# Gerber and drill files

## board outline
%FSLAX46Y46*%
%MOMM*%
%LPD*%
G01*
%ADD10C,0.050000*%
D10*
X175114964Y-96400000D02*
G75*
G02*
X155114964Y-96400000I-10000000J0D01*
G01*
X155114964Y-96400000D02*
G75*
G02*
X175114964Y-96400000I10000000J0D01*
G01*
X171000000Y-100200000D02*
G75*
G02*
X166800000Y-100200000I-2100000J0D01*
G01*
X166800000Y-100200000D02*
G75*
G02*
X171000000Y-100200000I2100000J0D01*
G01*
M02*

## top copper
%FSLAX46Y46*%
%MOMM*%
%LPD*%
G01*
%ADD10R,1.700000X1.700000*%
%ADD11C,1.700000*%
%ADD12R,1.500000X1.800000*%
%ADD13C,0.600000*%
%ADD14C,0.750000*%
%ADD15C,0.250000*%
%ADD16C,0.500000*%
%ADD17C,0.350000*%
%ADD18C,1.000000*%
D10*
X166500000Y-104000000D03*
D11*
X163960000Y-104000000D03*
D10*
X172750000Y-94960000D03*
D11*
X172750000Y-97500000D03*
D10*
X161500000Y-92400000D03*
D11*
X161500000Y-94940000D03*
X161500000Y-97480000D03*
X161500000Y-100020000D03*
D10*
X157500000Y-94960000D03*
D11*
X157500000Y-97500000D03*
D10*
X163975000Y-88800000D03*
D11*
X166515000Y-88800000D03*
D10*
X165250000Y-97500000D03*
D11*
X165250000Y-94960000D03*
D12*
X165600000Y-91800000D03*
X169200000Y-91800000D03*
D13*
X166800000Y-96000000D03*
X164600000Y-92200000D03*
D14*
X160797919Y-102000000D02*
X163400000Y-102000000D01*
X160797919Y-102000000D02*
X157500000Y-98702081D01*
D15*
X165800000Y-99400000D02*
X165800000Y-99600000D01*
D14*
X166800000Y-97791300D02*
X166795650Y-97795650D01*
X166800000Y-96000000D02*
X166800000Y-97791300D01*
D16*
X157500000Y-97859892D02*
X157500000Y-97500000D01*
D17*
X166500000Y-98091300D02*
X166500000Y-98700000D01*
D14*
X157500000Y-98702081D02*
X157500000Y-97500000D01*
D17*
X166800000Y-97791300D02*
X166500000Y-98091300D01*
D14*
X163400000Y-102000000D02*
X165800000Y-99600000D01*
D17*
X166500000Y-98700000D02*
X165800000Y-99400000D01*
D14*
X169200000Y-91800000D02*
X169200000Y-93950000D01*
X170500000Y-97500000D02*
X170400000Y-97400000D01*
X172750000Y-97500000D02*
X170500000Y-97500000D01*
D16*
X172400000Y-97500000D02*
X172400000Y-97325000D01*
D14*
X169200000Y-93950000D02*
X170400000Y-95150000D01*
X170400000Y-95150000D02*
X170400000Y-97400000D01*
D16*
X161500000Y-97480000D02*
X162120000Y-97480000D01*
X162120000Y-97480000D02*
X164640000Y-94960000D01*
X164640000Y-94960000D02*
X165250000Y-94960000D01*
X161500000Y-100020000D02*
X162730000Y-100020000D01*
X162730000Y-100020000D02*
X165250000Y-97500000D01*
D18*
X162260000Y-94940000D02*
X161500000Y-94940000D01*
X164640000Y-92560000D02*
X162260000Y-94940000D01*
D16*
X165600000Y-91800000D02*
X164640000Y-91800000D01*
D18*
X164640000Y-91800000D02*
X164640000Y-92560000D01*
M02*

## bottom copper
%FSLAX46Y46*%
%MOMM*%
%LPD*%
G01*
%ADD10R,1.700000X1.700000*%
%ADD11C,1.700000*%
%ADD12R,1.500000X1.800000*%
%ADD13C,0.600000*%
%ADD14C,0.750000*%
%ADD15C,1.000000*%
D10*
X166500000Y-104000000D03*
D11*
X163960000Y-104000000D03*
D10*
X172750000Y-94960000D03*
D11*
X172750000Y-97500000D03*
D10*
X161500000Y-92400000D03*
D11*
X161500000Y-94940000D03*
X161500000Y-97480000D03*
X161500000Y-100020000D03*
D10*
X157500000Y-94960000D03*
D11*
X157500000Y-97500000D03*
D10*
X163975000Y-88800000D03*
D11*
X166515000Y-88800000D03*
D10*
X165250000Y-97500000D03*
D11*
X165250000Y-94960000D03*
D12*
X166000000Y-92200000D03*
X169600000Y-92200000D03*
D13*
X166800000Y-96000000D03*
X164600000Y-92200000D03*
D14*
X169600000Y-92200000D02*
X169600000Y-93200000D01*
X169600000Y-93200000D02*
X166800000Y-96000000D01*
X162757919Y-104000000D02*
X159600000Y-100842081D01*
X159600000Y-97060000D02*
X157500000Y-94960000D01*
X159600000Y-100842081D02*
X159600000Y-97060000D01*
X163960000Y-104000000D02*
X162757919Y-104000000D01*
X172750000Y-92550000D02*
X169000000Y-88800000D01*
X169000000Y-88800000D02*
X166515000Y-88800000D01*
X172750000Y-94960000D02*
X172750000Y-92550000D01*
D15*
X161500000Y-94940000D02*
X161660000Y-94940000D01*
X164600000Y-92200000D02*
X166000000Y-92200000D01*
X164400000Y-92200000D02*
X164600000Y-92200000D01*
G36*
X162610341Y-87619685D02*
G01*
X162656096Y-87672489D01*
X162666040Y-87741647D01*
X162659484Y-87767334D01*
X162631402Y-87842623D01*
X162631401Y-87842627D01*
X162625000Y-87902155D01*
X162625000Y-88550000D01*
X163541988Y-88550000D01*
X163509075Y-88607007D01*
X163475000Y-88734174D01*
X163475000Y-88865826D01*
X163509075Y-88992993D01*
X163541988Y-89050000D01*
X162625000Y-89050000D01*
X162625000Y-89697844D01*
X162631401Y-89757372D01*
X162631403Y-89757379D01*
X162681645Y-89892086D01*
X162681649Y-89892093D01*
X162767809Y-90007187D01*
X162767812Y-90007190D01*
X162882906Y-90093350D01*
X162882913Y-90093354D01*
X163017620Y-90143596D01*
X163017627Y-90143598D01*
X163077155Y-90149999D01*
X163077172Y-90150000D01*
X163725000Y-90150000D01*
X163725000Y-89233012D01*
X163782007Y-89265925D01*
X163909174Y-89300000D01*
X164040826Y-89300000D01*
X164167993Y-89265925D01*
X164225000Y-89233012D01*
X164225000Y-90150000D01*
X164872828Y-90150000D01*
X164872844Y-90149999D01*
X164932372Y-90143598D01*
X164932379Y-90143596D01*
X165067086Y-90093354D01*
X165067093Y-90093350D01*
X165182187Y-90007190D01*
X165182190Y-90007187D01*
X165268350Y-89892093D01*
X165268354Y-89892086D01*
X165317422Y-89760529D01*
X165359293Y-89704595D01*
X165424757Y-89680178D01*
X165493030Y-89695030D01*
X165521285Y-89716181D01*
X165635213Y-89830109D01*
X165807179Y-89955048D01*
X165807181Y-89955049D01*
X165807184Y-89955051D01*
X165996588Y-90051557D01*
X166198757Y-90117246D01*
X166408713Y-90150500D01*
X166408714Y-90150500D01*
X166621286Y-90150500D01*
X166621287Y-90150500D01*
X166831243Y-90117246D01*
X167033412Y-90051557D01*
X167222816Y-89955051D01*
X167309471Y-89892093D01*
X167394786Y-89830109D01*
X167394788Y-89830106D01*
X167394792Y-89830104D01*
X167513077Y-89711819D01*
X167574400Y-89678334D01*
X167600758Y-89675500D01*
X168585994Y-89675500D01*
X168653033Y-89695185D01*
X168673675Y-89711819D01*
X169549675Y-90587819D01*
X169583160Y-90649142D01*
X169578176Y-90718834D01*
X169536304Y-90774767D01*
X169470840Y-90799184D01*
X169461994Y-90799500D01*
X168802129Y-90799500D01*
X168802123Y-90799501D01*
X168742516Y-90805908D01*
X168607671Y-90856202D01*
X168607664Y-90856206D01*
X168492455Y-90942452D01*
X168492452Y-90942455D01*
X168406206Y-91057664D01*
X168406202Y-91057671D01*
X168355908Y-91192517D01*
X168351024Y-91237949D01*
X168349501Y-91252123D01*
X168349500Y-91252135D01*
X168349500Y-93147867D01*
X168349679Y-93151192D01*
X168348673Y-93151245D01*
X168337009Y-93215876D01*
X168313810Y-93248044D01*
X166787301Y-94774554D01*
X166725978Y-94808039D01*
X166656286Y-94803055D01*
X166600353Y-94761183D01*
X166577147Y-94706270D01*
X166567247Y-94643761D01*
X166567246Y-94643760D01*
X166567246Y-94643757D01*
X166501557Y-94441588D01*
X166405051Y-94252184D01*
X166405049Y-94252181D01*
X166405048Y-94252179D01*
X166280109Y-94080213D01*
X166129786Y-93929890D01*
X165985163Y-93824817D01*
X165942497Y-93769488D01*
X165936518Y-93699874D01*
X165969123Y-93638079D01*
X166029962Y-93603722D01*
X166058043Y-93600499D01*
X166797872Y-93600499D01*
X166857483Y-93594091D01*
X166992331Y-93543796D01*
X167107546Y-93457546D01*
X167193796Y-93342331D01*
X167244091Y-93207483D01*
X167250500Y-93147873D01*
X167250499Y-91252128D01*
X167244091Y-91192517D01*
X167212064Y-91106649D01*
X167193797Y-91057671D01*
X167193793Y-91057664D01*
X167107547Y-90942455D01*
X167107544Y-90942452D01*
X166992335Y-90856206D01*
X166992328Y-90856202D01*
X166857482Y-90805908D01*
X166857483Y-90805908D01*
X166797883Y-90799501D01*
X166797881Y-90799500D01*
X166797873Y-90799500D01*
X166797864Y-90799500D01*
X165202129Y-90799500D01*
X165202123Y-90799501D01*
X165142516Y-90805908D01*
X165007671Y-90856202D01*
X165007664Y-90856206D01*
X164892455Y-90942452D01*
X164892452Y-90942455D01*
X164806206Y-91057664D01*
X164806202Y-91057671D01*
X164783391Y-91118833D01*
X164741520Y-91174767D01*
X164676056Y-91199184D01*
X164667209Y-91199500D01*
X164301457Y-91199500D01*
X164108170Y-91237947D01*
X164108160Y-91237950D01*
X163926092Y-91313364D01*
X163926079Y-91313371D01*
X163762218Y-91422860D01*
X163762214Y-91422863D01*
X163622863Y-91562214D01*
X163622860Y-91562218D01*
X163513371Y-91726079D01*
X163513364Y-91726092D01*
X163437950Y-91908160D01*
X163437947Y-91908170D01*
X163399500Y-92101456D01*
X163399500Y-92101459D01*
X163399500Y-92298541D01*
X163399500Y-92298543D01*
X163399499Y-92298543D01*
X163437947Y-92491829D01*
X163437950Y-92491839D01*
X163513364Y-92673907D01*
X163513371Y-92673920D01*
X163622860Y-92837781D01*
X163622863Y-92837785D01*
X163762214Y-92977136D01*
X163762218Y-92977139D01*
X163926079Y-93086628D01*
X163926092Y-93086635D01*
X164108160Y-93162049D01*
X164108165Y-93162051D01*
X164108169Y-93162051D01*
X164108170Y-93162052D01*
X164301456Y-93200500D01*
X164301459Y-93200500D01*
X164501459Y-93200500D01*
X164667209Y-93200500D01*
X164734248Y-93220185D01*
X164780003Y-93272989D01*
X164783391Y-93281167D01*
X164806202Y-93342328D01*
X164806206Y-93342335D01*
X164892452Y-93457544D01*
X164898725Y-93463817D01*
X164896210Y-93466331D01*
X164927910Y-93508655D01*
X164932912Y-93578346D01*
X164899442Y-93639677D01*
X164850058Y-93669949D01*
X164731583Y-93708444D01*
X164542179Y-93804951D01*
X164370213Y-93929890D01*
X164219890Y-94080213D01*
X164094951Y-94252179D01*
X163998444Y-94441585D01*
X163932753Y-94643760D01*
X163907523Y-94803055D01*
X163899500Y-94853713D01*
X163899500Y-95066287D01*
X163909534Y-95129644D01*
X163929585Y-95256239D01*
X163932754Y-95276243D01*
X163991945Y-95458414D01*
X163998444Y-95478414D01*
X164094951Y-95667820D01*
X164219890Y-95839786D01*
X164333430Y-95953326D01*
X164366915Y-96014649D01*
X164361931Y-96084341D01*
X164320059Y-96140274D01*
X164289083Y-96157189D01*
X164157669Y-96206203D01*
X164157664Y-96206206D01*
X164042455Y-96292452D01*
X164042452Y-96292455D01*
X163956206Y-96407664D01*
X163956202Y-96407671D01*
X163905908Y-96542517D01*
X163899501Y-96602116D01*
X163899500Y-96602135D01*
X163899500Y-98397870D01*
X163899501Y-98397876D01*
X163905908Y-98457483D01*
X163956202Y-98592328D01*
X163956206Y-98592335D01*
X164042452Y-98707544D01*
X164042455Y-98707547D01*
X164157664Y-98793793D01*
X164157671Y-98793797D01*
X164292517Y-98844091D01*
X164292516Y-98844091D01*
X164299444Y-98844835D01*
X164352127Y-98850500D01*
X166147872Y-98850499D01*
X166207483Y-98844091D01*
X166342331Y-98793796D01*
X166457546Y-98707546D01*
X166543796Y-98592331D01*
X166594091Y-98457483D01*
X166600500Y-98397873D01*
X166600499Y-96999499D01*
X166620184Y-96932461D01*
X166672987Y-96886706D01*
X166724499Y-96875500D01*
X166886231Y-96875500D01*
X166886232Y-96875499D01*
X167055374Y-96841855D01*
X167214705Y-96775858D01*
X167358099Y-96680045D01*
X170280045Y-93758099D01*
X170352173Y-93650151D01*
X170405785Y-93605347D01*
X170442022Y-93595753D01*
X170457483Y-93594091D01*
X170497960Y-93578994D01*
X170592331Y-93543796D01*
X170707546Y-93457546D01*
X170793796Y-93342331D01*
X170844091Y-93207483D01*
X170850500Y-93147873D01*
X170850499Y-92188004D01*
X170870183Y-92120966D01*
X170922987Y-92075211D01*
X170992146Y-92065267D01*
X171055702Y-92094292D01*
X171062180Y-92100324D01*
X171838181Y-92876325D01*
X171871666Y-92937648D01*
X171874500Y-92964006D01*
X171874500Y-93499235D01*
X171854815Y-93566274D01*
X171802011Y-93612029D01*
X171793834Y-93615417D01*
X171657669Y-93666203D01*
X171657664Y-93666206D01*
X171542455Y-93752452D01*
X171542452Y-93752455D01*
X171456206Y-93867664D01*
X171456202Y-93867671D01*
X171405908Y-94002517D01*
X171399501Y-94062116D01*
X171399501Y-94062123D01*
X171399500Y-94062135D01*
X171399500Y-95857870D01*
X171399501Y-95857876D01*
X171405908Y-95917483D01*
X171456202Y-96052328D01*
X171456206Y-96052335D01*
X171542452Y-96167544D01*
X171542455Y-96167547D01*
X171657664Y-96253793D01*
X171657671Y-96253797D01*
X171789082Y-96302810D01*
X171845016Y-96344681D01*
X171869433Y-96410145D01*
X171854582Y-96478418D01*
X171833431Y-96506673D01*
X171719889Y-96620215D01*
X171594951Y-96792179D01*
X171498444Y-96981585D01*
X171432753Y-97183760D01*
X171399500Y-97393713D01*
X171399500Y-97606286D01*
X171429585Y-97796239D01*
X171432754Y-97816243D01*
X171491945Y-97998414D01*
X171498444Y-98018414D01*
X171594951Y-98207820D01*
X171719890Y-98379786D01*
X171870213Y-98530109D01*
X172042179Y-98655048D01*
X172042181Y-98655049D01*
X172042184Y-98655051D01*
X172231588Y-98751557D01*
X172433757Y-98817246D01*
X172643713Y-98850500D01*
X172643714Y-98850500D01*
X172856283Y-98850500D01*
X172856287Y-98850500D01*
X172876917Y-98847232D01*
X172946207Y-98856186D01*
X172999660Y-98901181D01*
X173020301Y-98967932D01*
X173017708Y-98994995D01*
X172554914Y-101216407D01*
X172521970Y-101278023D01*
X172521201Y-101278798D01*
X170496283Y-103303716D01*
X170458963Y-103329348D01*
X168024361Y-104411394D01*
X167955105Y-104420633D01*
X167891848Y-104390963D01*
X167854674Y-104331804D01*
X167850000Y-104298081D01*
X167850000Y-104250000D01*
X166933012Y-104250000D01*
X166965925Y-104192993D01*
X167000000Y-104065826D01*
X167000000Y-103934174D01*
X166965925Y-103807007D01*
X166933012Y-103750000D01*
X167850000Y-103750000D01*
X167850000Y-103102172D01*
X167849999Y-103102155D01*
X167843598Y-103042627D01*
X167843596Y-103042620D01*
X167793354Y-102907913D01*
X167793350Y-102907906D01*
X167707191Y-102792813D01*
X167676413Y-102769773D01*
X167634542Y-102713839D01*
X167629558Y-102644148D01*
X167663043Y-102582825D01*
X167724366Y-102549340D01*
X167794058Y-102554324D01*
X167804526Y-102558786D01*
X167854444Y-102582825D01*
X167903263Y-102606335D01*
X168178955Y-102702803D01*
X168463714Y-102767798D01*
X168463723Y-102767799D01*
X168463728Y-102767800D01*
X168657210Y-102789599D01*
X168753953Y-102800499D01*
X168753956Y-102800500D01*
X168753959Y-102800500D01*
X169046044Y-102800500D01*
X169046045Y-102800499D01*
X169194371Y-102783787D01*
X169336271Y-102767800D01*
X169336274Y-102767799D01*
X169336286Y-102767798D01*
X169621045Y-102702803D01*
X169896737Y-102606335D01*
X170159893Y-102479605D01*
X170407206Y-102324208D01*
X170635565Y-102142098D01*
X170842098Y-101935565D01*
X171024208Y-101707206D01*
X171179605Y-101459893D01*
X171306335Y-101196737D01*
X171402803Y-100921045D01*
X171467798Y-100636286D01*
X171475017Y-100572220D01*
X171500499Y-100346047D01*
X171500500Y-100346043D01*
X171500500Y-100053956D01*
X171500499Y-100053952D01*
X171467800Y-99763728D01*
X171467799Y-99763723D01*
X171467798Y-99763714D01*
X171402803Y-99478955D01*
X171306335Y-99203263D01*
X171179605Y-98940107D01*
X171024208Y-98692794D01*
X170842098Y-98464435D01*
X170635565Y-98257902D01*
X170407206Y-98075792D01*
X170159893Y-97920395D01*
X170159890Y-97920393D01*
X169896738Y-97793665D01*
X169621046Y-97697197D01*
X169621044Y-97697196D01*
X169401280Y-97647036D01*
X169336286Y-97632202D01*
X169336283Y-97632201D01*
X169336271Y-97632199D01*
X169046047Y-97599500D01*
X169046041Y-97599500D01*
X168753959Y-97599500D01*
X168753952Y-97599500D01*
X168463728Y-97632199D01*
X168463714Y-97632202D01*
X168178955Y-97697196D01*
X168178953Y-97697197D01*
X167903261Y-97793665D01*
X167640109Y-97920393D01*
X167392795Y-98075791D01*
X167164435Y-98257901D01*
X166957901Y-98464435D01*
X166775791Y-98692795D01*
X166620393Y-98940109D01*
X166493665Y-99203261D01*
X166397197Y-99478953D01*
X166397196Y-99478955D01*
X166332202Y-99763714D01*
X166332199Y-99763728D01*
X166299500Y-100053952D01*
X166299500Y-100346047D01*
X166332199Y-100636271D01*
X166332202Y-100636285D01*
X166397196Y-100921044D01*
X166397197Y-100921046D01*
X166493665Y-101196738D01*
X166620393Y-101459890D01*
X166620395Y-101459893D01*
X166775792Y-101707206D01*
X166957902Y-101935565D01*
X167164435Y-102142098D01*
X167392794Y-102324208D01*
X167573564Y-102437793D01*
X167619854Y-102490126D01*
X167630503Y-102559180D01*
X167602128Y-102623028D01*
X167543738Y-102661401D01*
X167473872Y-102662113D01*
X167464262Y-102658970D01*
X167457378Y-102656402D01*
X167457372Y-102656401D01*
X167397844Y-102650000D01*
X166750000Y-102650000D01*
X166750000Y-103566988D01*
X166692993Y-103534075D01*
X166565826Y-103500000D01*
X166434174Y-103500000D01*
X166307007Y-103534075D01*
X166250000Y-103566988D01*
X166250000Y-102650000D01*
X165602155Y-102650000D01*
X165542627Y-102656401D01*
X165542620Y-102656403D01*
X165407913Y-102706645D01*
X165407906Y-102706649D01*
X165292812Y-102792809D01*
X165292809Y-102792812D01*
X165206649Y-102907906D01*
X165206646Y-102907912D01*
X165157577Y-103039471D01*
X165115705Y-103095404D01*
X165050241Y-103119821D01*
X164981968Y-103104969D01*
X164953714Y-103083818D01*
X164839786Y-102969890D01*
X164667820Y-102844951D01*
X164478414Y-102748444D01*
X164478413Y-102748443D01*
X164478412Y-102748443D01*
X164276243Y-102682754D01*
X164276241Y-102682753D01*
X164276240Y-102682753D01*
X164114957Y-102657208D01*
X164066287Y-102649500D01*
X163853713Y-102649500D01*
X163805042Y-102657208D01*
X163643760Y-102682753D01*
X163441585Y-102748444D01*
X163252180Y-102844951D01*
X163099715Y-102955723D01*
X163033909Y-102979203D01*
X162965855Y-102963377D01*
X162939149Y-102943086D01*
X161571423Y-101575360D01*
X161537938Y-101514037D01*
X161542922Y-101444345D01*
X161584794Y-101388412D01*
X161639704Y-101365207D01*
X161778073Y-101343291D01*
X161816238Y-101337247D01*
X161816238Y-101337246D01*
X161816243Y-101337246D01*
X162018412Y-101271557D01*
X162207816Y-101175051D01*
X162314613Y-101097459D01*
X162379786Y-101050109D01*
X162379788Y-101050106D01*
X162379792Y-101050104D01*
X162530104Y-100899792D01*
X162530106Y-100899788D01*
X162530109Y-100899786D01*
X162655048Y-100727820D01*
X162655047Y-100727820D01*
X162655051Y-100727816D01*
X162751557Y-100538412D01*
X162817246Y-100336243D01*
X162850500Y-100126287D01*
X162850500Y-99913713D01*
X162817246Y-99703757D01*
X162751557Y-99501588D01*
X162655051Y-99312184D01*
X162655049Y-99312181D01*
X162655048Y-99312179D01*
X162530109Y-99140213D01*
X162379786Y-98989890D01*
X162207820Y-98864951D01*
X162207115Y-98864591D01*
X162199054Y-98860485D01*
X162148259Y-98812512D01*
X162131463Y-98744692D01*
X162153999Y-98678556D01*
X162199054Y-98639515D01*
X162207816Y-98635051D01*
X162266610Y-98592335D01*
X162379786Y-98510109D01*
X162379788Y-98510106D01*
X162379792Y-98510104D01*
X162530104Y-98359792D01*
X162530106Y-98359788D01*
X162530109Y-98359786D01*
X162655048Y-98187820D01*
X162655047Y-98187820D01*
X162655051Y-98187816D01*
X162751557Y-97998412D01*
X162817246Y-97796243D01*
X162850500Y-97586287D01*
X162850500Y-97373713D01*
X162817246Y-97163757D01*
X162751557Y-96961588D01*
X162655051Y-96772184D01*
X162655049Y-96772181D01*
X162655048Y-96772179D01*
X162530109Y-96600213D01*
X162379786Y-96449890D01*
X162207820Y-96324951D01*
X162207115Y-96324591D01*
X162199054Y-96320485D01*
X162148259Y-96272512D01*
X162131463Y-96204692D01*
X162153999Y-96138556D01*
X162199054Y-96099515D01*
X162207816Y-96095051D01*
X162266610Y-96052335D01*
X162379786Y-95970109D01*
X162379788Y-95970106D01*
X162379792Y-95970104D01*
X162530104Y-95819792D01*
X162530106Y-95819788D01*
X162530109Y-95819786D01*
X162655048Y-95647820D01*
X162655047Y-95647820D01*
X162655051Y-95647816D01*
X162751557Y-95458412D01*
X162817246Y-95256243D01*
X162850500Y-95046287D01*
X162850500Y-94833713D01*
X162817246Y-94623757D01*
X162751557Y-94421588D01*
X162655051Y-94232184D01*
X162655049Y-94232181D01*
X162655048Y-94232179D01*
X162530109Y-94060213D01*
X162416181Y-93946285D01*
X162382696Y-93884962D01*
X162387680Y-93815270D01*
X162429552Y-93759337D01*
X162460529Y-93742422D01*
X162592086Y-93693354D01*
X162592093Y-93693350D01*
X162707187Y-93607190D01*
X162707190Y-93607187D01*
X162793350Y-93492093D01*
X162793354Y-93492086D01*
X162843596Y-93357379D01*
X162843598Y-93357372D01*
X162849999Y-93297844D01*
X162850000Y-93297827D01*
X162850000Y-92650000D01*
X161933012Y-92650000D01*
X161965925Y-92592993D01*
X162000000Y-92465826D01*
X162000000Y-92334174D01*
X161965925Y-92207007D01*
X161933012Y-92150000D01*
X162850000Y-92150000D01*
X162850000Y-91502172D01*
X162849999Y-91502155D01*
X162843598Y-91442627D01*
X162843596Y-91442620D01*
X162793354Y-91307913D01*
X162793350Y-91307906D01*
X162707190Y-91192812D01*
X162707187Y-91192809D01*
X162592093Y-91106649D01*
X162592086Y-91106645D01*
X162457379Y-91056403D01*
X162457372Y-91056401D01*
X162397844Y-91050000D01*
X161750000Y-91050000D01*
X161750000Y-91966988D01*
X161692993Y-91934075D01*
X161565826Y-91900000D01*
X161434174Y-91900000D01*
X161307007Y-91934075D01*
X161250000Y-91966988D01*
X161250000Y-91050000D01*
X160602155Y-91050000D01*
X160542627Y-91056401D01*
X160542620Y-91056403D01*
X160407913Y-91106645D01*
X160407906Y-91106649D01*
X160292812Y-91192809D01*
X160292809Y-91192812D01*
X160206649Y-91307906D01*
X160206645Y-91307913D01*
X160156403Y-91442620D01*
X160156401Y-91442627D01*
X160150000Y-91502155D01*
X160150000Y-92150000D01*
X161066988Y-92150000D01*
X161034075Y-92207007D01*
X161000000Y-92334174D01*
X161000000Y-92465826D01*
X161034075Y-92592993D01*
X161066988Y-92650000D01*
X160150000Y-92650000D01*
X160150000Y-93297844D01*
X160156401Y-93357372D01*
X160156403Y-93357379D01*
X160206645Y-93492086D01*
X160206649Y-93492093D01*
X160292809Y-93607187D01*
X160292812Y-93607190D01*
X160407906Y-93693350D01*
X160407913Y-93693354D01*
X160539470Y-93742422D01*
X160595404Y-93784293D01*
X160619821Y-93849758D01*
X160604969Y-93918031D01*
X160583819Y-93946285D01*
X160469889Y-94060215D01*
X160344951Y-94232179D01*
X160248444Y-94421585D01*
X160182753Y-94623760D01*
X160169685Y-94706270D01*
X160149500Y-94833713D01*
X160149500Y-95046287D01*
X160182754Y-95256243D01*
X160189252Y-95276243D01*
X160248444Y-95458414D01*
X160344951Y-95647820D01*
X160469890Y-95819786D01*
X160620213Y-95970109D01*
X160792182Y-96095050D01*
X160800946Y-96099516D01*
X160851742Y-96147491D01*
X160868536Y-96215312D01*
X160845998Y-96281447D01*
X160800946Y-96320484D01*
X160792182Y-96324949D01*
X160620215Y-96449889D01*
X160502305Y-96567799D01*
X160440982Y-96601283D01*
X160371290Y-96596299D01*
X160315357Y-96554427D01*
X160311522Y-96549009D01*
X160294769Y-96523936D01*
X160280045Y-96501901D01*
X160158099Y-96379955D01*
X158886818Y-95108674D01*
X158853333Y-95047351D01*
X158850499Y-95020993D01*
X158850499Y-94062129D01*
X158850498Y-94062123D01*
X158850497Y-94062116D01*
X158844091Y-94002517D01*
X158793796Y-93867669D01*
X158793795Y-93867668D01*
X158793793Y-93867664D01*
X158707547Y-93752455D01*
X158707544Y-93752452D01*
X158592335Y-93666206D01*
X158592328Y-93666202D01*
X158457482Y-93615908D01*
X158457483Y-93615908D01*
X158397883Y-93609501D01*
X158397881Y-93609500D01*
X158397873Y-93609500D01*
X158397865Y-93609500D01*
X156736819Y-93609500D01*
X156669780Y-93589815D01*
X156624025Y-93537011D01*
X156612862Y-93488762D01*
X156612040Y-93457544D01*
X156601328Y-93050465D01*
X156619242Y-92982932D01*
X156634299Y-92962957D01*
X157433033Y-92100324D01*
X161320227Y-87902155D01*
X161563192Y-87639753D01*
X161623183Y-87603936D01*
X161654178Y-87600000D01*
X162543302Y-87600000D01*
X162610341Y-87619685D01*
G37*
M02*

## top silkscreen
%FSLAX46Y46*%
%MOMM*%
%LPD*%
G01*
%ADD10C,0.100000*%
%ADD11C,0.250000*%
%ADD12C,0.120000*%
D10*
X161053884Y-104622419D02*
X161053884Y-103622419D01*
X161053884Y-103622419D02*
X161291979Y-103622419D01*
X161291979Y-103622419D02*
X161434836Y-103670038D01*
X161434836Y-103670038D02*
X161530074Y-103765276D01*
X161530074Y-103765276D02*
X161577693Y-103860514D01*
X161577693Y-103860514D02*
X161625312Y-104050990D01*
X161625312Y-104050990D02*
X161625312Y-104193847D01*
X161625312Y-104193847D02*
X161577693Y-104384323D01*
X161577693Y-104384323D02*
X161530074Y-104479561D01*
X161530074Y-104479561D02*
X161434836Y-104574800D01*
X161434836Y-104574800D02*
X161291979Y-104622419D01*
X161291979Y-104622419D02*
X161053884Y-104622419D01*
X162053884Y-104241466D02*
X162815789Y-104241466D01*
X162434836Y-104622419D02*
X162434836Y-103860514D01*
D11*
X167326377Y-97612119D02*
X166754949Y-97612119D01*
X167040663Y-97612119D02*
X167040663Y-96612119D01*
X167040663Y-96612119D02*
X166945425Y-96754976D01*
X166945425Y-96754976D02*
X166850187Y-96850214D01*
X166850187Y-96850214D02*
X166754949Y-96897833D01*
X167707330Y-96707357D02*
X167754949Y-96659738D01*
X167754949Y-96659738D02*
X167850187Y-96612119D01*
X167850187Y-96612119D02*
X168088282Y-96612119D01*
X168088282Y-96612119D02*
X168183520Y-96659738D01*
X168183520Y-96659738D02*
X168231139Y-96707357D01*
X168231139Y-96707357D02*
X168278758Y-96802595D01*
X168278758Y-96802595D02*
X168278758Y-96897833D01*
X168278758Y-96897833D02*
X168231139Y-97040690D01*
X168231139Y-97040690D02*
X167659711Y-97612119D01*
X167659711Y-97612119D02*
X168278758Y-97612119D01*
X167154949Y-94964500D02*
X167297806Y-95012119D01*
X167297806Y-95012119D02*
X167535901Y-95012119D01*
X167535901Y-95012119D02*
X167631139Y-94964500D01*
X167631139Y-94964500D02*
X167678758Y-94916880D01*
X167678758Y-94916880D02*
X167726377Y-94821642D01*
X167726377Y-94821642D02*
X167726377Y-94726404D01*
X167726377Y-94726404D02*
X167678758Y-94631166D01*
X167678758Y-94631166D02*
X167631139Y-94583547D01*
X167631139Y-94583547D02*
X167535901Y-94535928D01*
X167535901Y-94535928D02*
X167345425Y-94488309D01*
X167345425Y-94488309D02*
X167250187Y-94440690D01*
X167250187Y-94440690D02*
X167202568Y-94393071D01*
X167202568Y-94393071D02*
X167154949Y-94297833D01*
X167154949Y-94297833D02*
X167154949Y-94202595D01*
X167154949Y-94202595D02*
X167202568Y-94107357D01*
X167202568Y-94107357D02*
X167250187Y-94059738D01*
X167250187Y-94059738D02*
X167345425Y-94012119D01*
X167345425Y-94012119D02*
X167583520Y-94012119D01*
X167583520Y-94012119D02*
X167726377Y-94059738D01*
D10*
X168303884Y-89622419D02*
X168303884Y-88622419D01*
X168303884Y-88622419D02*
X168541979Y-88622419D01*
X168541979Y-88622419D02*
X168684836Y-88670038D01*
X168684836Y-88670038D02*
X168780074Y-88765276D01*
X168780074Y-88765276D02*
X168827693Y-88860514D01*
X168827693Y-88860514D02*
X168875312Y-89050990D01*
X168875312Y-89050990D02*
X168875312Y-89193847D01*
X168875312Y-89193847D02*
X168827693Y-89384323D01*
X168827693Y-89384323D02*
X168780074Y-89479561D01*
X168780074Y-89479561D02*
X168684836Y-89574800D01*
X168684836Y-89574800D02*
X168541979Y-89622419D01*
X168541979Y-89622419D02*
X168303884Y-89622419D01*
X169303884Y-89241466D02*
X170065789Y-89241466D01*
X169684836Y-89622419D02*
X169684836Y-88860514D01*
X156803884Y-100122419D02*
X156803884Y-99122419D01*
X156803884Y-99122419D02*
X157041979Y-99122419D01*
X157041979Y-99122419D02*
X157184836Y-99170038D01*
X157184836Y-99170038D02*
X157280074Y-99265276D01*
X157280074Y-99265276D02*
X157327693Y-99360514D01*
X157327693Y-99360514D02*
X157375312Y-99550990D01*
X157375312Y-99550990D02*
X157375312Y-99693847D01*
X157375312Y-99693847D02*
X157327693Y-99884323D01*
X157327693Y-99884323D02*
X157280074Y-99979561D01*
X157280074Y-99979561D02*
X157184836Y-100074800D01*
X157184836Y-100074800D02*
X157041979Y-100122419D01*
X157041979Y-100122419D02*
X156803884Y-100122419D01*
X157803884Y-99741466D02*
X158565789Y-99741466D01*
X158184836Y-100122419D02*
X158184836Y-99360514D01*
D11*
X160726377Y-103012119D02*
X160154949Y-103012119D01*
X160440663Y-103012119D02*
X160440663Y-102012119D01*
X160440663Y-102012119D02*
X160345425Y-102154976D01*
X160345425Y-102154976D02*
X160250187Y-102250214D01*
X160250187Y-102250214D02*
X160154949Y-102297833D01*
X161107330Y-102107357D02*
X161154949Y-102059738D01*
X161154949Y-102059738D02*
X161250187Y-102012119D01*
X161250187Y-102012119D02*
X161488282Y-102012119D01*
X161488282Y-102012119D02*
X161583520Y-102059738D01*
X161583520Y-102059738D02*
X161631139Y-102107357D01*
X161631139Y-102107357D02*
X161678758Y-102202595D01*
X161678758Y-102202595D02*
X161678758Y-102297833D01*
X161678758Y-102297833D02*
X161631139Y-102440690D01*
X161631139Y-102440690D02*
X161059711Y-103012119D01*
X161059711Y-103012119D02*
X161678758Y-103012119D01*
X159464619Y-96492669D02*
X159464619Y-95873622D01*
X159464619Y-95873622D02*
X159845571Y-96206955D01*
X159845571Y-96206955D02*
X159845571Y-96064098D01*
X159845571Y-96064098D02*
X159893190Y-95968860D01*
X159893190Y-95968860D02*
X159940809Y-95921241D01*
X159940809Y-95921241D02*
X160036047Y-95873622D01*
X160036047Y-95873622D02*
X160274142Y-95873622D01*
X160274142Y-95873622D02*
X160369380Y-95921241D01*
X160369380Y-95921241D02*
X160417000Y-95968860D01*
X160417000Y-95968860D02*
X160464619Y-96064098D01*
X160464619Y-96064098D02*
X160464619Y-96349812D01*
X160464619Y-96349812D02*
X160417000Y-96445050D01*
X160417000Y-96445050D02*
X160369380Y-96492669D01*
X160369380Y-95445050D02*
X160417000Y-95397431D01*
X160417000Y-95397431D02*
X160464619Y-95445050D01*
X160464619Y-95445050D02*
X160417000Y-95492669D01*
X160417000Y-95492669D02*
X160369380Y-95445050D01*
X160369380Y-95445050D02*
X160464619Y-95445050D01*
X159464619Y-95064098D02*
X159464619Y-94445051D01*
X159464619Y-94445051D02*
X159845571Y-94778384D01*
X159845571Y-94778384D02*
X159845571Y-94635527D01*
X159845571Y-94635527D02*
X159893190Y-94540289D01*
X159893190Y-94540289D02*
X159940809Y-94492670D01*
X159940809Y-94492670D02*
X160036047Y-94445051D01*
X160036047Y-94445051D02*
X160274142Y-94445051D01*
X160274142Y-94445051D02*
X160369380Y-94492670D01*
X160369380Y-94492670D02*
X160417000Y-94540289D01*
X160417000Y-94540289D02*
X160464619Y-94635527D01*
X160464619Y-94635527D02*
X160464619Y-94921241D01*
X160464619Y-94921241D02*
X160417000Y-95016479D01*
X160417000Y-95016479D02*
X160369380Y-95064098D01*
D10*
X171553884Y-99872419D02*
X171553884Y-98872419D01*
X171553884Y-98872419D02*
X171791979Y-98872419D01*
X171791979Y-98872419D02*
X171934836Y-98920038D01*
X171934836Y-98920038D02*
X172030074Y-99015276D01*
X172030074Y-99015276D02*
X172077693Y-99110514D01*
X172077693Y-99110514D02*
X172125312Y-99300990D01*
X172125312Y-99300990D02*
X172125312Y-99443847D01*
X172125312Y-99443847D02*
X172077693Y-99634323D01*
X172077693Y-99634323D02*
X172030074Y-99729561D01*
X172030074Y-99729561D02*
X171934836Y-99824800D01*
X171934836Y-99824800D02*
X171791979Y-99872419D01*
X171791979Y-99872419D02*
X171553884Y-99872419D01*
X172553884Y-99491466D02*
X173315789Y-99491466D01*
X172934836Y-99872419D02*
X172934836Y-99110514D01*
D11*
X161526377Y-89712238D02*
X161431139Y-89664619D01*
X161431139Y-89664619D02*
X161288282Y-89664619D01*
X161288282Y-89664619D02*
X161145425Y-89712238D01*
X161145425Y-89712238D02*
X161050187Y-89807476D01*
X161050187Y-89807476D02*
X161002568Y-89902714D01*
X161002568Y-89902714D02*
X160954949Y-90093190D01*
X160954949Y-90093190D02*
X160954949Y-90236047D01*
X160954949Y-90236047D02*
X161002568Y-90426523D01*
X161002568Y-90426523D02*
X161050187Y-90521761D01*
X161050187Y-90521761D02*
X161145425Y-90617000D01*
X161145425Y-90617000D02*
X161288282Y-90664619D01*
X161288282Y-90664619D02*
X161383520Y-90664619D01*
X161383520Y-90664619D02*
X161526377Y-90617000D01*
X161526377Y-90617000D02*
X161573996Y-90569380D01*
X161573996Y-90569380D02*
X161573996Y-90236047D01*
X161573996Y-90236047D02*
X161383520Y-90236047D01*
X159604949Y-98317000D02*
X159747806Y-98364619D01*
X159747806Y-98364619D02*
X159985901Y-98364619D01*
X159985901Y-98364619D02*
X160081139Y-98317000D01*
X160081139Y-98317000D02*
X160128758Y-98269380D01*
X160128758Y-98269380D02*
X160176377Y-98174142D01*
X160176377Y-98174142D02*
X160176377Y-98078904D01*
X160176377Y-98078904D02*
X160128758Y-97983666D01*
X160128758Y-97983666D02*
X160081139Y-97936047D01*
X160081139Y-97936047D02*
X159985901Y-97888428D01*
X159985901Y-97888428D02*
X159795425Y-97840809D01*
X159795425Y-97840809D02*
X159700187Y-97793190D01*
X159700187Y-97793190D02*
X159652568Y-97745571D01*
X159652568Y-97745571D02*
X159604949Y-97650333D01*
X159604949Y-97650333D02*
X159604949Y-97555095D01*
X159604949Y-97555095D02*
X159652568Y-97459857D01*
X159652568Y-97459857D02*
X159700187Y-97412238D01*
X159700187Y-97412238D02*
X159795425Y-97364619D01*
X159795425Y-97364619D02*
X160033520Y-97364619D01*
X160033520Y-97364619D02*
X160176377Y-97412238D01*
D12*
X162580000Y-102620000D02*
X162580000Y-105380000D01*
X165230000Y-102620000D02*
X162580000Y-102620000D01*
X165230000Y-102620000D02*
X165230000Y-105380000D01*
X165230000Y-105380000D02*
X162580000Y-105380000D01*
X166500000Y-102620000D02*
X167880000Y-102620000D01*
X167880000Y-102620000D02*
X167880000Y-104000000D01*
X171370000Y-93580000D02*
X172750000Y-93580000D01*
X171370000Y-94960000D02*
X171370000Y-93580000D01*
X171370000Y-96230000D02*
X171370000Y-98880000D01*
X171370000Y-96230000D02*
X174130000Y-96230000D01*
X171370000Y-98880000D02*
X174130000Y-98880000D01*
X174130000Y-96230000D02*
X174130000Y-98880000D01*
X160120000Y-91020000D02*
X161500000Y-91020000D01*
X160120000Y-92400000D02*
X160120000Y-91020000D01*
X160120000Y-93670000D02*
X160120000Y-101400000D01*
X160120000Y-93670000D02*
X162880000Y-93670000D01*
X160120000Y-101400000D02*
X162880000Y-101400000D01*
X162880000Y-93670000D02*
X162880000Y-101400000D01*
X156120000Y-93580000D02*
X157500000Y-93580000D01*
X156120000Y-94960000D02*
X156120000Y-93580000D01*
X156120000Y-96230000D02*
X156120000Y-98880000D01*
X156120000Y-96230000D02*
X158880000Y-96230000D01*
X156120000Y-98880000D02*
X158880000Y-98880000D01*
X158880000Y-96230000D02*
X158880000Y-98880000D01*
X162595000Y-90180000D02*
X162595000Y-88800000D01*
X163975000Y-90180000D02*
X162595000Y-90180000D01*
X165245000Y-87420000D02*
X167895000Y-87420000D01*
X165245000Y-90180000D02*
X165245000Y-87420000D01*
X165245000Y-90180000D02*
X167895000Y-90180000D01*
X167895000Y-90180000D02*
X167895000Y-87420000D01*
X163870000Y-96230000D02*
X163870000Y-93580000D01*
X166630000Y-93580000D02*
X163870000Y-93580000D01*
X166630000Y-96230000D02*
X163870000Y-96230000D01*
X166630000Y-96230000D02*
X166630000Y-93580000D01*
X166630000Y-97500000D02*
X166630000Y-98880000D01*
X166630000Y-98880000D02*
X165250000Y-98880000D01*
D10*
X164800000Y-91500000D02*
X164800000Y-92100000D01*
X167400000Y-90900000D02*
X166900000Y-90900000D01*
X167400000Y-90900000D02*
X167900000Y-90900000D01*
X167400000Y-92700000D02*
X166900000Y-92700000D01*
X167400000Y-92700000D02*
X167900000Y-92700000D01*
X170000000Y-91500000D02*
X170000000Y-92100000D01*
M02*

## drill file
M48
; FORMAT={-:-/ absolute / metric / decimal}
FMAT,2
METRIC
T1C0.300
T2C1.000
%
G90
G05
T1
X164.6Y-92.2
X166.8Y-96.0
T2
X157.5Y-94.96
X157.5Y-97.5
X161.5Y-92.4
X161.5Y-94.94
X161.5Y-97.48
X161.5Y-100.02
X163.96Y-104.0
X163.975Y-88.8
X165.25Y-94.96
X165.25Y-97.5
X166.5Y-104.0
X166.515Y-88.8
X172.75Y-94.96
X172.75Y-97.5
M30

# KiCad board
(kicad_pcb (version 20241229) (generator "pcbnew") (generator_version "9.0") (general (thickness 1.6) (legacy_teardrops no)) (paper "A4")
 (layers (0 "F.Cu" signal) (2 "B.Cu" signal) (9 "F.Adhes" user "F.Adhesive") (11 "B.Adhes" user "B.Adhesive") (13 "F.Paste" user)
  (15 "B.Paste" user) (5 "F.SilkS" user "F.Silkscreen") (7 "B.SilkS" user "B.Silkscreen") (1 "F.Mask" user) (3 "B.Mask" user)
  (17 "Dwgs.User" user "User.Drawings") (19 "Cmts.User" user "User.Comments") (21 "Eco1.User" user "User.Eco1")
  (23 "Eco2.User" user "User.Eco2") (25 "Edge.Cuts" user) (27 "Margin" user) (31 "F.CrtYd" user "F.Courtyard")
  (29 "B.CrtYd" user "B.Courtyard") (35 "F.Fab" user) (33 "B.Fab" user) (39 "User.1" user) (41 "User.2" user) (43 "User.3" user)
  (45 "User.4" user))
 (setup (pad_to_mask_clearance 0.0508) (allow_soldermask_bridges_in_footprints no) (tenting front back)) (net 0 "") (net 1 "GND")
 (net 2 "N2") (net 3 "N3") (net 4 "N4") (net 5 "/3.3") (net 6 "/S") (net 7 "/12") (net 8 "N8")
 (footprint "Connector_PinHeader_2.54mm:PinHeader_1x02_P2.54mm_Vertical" (layer "F.Cu") (at 166.5 104 -90)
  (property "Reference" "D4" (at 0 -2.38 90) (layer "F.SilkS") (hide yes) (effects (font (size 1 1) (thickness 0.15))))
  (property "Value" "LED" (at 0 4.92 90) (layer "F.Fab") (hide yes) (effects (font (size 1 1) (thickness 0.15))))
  (fp_line (start -1.38 3.92) (end 1.38 3.92) (stroke (width 0.12) (type solid)) (layer "F.SilkS"))
  (fp_line (start -1.38 1.27) (end -1.38 3.92) (stroke (width 0.12) (type solid)) (layer "F.SilkS"))
  (fp_line (start -1.38 1.27) (end 1.38 1.27) (stroke (width 0.12) (type solid)) (layer "F.SilkS"))
  (fp_line (start 1.38 1.27) (end 1.38 3.92) (stroke (width 0.12) (type solid)) (layer "F.SilkS"))
  (fp_line (start -1.38 0) (end -1.38 -1.38) (stroke (width 0.12) (type solid)) (layer "F.SilkS"))
  (fp_line (start -1.38 -1.38) (end 0 -1.38) (stroke (width 0.12) (type solid)) (layer "F.SilkS"))
  (pad "1" thru_hole rect (at 0 0 270) (size 1.7 1.7) (drill 1) (layers "*.Cu" "*.Mask") (remove_unused_layers no) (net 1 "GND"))
  (pad "2" thru_hole circle (at 0 2.54 270) (size 1.7 1.7) (drill 1) (layers "*.Cu" "*.Mask") (remove_unused_layers no) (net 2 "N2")))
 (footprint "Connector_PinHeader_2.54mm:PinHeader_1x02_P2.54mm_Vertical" (layer "F.Cu") (at 172.75 94.96)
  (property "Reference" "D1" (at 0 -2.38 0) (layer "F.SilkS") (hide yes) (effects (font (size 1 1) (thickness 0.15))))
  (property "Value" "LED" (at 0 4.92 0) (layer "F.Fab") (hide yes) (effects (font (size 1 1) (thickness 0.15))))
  (fp_line (start -1.38 -1.38) (end 0 -1.38) (stroke (width 0.12) (type solid)) (layer "F.SilkS"))
  (fp_line (start -1.38 0) (end -1.38 -1.38) (stroke (width 0.12) (type solid)) (layer "F.SilkS"))
  (fp_line (start -1.38 1.27) (end -1.38 3.92) (stroke (width 0.12) (type solid)) (layer "F.SilkS"))
  (fp_line (start -1.38 1.27) (end 1.38 1.27) (stroke (width 0.12) (type solid)) (layer "F.SilkS"))
  (fp_line (start -1.38 3.92) (end 1.38 3.92) (stroke (width 0.12) (type solid)) (layer "F.SilkS"))
  (fp_line (start 1.38 1.27) (end 1.38 3.92) (stroke (width 0.12) (type solid)) (layer "F.SilkS"))
  (pad "1" thru_hole rect (at 0 0) (size 1.7 1.7) (drill 1) (layers "*.Cu" "*.Mask") (remove_unused_layers no) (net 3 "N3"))
  (pad "2" thru_hole circle (at 0 2.54) (size 1.7 1.7) (drill 1) (layers "*.Cu" "*.Mask") (remove_unused_layers no) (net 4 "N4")))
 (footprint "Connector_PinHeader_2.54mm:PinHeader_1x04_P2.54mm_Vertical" (layer "F.Cu") (at 161.5 92.4)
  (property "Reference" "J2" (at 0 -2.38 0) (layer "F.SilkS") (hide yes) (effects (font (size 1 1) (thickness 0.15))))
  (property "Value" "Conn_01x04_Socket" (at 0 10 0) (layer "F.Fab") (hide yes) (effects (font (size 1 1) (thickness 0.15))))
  (fp_line (start -1.38 -1.38) (end 0 -1.38) (stroke (width 0.12) (type solid)) (layer "F.SilkS"))
  (fp_line (start -1.38 0) (end -1.38 -1.38) (stroke (width 0.12) (type solid)) (layer "F.SilkS"))
  (fp_line (start -1.38 1.27) (end -1.38 9) (stroke (width 0.12) (type solid)) (layer "F.SilkS"))
  (fp_line (start -1.38 1.27) (end 1.38 1.27) (stroke (width 0.12) (type solid)) (layer "F.SilkS"))
  (fp_line (start -1.38 9) (end 1.38 9) (stroke (width 0.12) (type solid)) (layer "F.SilkS"))
  (fp_line (start 1.38 1.27) (end 1.38 9) (stroke (width 0.12) (type solid)) (layer "F.SilkS"))
  (pad "1" thru_hole rect (at 0 0) (size 1.7 1.7) (drill 1) (layers "*.Cu" "*.Mask") (remove_unused_layers no) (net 1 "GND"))
  (pad "2" thru_hole circle (at 0 2.54) (size 1.7 1.7) (drill 1) (layers "*.Cu" "*.Mask") (remove_unused_layers no) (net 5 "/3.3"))
  (pad "3" thru_hole circle (at 0 5.08) (size 1.7 1.7) (drill 1) (layers "*.Cu" "*.Mask") (remove_unused_layers no) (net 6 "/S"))
  (pad "4" thru_hole circle (at 0 7.62) (size 1.7 1.7) (drill 1) (layers "*.Cu" "*.Mask") (remove_unused_layers no) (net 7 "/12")))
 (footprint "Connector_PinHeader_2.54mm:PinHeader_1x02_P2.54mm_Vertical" (layer "F.Cu") (at 157.5 94.96)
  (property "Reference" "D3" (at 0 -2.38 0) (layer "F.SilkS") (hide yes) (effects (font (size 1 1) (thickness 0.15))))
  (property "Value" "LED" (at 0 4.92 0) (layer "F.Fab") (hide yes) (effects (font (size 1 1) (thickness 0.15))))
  (fp_line (start -1.38 -1.38) (end 0 -1.38) (stroke (width 0.12) (type solid)) (layer "F.SilkS"))
  (fp_line (start -1.38 0) (end -1.38 -1.38) (stroke (width 0.12) (type solid)) (layer "F.SilkS"))
  (fp_line (start -1.38 1.27) (end -1.38 3.92) (stroke (width 0.12) (type solid)) (layer "F.SilkS"))
  (fp_line (start -1.38 1.27) (end 1.38 1.27) (stroke (width 0.12) (type solid)) (layer "F.SilkS"))
  (fp_line (start -1.38 3.92) (end 1.38 3.92) (stroke (width 0.12) (type solid)) (layer "F.SilkS"))
  (fp_line (start 1.38 1.27) (end 1.38 3.92) (stroke (width 0.12) (type solid)) (layer "F.SilkS"))
  (pad "1" thru_hole rect (at 0 0) (size 1.7 1.7) (drill 1) (layers "*.Cu" "*.Mask") (remove_unused_layers no) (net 2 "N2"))
  (pad "2" thru_hole circle (at 0 2.54) (size 1.7 1.7) (drill 1) (layers "*.Cu" "*.Mask") (remove_unused_layers no) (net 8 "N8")))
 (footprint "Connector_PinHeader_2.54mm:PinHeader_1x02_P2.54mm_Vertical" (layer "F.Cu") (at 163.975 88.8 90)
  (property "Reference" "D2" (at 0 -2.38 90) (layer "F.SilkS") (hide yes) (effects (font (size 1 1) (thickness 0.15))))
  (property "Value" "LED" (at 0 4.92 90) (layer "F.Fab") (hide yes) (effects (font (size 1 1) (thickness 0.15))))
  (fp_line (start -1.38 -1.38) (end 0 -1.38) (stroke (width 0.12) (type solid)) (layer "F.SilkS"))
  (fp_line (start -1.38 0) (end -1.38 -1.38) (stroke (width 0.12) (type solid)) (layer "F.SilkS"))
  (fp_line (start 1.38 1.27) (end 1.38 3.92) (stroke (width 0.12) (type solid)) (layer "F.SilkS"))
  (fp_line (start -1.38 1.27) (end 1.38 1.27) (stroke (width 0.12) (type solid)) (layer "F.SilkS"))
  (fp_line (start -1.38 1.27) (end -1.38 3.92) (stroke (width 0.12) (type solid)) (layer "F.SilkS"))
  (fp_line (start -1.38 3.92) (end 1.38 3.92) (stroke (width 0.12) (type solid)) (layer "F.SilkS"))
  (pad "1" thru_hole rect (at 0 0 90) (size 1.7 1.7) (drill 1) (layers "*.Cu" "*.Mask") (remove_unused_layers no) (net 1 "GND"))
  (pad "2" thru_hole circle (at 0 2.54 90) (size 1.7 1.7) (drill 1) (layers "*.Cu" "*.Mask") (remove_unused_layers no) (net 3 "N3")))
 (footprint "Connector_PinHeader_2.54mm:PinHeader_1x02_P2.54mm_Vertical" (layer "F.Cu") (at 165.25 97.5 180)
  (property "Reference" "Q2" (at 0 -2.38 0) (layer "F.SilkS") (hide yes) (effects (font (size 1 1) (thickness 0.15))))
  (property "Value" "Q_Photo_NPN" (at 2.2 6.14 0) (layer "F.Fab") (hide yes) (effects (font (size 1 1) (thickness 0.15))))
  (fp_line (start 1.38 1.27) (end 1.38 3.92) (stroke (width 0.12) (type solid)) (layer "F.SilkS"))
  (fp_line (start -1.38 3.92) (end 1.38 3.92) (stroke (width 0.12) (type solid)) (layer "F.SilkS"))
  (fp_line (start -1.38 1.27) (end 1.38 1.27) (stroke (width 0.12) (type solid)) (layer "F.SilkS"))
  (fp_line (start -1.38 1.27) (end -1.38 3.92) (stroke (width 0.12) (type solid)) (layer "F.SilkS"))
  (fp_line (start -1.38 0) (end -1.38 -1.38) (stroke (width 0.12) (type solid)) (layer "F.SilkS"))
  (fp_line (start -1.38 -1.38) (end 0 -1.38) (stroke (width 0.12) (type solid)) (layer "F.SilkS"))
  (pad "1" thru_hole rect (at 0 0 180) (size 1.7 1.7) (drill 1) (layers "*.Cu" "*.Mask") (remove_unused_layers no) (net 7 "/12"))
  (pad "2" thru_hole circle (at 0 2.54 180) (size 1.7 1.7) (drill 1) (layers "*.Cu" "*.Mask") (remove_unused_layers no) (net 6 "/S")))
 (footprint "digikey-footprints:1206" (layer "F.Cu") (at 167.4 91.8)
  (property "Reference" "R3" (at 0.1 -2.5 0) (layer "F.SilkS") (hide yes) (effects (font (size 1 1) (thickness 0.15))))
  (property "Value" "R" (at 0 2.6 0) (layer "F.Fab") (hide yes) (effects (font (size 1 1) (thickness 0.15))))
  (fp_line (start -2.6 -0.3) (end -2.6 0.3) (stroke (width 0.1) (type solid)) (layer "F.SilkS"))
  (fp_line (start 0 -0.9) (end -0.5 -0.9) (stroke (width 0.1) (type solid)) (layer "F.SilkS"))
  (fp_line (start 0 -0.9) (end 0.5 -0.9) (stroke (width 0.1) (type solid)) (layer "F.SilkS"))
  (fp_line (start 0 0.9) (end -0.5 0.9) (stroke (width 0.1) (type solid)) (layer "F.SilkS"))
  (fp_line (start 0 0.9) (end 0.5 0.9) (stroke (width 0.1) (type solid)) (layer "F.SilkS"))
  (fp_line (start 2.6 -0.3) (end 2.6 0.3) (stroke (width 0.1) (type solid)) (layer "F.SilkS"))
  (pad "1" smd rect (at -1.8 0) (size 1.5 1.8) (layers "F.Cu" "F.Mask" "F.Paste") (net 5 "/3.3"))
  (pad "2" smd rect (at 1.8 0) (size 1.5 1.8) (layers "F.Cu" "F.Mask" "F.Paste") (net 4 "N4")))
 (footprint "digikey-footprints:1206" (layer "B.Cu") (at 167.8 92.2)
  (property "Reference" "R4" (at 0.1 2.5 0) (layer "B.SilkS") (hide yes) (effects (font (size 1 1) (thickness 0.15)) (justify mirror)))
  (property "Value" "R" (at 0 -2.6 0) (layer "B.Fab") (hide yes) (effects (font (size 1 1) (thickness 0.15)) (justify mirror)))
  (pad "1" smd rect (at -1.8 0) (size 1.5 1.8) (layers "B.Cu" "B.Mask" "B.Paste") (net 5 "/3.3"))
  (pad "2" smd rect (at 1.8 0) (size 1.5 1.8) (layers "B.Cu" "B.Mask" "B.Paste") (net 8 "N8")))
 (gr_circle (center 165.114964 96.4) (end 175.114964 96.4) (stroke (width 0.05) (type solid)) (fill no) (layer "Edge.Cuts"))
 (gr_circle (center 168.9 100.2) (end 171 100.2) (stroke (width 0.05) (type solid)) (fill no) (layer "Edge.Cuts"))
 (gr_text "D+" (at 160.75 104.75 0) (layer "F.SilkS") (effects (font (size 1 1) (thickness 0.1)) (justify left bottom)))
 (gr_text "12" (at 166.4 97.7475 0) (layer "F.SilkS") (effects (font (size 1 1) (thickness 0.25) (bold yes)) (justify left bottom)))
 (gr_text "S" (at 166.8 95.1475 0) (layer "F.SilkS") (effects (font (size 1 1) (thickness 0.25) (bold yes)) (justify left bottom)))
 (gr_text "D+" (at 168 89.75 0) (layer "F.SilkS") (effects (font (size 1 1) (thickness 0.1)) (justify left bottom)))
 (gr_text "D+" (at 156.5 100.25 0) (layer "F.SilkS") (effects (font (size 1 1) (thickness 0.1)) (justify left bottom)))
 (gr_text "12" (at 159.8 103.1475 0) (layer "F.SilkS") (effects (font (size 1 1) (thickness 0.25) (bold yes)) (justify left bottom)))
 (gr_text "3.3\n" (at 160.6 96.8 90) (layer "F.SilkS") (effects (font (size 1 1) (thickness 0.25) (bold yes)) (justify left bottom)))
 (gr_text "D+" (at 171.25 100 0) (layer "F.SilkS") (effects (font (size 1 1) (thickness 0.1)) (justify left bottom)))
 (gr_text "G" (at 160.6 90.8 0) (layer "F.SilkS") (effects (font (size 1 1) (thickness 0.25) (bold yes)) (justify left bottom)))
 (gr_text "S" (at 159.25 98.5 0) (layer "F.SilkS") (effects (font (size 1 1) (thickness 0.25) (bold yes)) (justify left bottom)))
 (segment (start 160.797919 102) (end 163.4 102) (width 0.75) (layer "F.Cu") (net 8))
 (segment (start 160.797919 102) (end 157.5 98.702081) (width 0.75) (layer "F.Cu") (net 8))
 (segment (start 165.8 99.4) (end 165.8 99.6) (width 0.25) (layer "F.Cu") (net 8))
 (segment (start 166.8 97.7913) (end 166.79565 97.79565) (width 0.75) (layer "F.Cu") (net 8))
 (segment (start 166.8 96) (end 166.8 97.7913) (width 0.75) (layer "F.Cu") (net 8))
 (segment (start 157.5 97.859892) (end 157.5 97.5) (width 0.5) (layer "F.Cu") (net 8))
 (segment (start 166.5 98.0913) (end 166.5 98.7) (width 0.35) (layer "F.Cu") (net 8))
 (segment (start 157.5 98.702081) (end 157.5 97.5) (width 0.75) (layer "F.Cu") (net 8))
 (segment (start 166.8 97.7913) (end 166.5 98.0913) (width 0.35) (layer "F.Cu") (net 8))
 (segment (start 163.4 102) (end 165.8 99.6) (width 0.75) (layer "F.Cu") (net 8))
 (segment (start 166.5 98.7) (end 165.8 99.4) (width 0.35) (layer "F.Cu") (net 8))
 (via (at 166.8 96) (size 0.6) (drill 0.3) (layers "F.Cu" "B.Cu") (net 8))
 (segment (start 169.6 92.2) (end 169.6 93.2) (width 0.75) (layer "B.Cu") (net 8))
 (segment (start 169.6 93.2) (end 166.8 96) (width 0.75) (layer "B.Cu") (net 8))
 (segment (start 162.757919 104) (end 159.6 100.842081) (width 0.75) (layer "B.Cu") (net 2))
 (segment (start 159.6 97.06) (end 157.5 94.96) (width 0.75) (layer "B.Cu") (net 2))
 (segment (start 159.6 100.842081) (end 159.6 97.06) (width 0.75) (layer "B.Cu") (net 2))
 (segment (start 163.96 104) (end 162.757919 104) (width 0.75) (layer "B.Cu") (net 2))
 (segment (start 172.75 92.55) (end 169 88.8) (width 0.75) (layer "B.Cu") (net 3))
 (segment (start 169 88.8) (end 166.515 88.8) (width 0.75) (layer "B.Cu") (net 3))
 (segment (start 172.75 94.96) (end 172.75 92.55) (width 0.75) (layer "B.Cu") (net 3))
 (segment (start 169.2 91.8) (end 169.2 93.95) (width 0.75) (layer "F.Cu") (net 4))
 (segment (start 170.5 97.5) (end 170.4 97.4) (width 0.75) (layer "F.Cu") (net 4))
 (segment (start 172.75 97.5) (end 170.5 97.5) (width 0.75) (layer "F.Cu") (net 4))
 (segment (start 172.4 97.5) (end 172.4 97.325) (width 0.5) (layer "F.Cu") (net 4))
 (segment (start 169.2 93.95) (end 170.4 95.15) (width 0.75) (layer "F.Cu") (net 4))
 (segment (start 170.4 95.15) (end 170.4 97.4) (width 0.75) (layer "F.Cu") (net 4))
 (segment (start 161.5 97.48) (end 162.12 97.48) (width 0.5) (layer "F.Cu") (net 6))
 (segment (start 162.12 97.48) (end 164.64 94.96) (width 0.5) (layer "F.Cu") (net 6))
 (segment (start 164.64 94.96) (end 165.25 94.96) (width 0.5) (layer "F.Cu") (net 6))
 (segment (start 161.5 100.02) (end 162.73 100.02) (width 0.5) (layer "F.Cu") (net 7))
 (segment (start 162.73 100.02) (end 165.25 97.5) (width 0.5) (layer "F.Cu") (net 7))
 (segment (start 162.26 94.94) (end 161.5 94.94) (width 1) (layer "F.Cu") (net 5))
 (segment (start 164.64 92.56) (end 162.26 94.94) (width 1) (layer "F.Cu") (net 5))
 (segment (start 165.6 91.8) (end 164.64 91.8) (width 0.5) (layer "F.Cu") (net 5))
 (segment (start 164.64 91.8) (end 164.64 92.56) (width 1) (layer "F.Cu") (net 5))
 (via (at 164.6 92.2) (size 0.6) (drill 0.3) (layers "F.Cu" "B.Cu") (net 5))
 (segment (start 161.5 94.94) (end 161.66 94.94) (width 1) (layer "B.Cu") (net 5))
 (segment (start 164.6 92.2) (end 166 92.2) (width 1) (layer "B.Cu") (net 5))
 (segment (start 164.4 92.2) (end 164.6 92.2) (width 1) (layer "B.Cu") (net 5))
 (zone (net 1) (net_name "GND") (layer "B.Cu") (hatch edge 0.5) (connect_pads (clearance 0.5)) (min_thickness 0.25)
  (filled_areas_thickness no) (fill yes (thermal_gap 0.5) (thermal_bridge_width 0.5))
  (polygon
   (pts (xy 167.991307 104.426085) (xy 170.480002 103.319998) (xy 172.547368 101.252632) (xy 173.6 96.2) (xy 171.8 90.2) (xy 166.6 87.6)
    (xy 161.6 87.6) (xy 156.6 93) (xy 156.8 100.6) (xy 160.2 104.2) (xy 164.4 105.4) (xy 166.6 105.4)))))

